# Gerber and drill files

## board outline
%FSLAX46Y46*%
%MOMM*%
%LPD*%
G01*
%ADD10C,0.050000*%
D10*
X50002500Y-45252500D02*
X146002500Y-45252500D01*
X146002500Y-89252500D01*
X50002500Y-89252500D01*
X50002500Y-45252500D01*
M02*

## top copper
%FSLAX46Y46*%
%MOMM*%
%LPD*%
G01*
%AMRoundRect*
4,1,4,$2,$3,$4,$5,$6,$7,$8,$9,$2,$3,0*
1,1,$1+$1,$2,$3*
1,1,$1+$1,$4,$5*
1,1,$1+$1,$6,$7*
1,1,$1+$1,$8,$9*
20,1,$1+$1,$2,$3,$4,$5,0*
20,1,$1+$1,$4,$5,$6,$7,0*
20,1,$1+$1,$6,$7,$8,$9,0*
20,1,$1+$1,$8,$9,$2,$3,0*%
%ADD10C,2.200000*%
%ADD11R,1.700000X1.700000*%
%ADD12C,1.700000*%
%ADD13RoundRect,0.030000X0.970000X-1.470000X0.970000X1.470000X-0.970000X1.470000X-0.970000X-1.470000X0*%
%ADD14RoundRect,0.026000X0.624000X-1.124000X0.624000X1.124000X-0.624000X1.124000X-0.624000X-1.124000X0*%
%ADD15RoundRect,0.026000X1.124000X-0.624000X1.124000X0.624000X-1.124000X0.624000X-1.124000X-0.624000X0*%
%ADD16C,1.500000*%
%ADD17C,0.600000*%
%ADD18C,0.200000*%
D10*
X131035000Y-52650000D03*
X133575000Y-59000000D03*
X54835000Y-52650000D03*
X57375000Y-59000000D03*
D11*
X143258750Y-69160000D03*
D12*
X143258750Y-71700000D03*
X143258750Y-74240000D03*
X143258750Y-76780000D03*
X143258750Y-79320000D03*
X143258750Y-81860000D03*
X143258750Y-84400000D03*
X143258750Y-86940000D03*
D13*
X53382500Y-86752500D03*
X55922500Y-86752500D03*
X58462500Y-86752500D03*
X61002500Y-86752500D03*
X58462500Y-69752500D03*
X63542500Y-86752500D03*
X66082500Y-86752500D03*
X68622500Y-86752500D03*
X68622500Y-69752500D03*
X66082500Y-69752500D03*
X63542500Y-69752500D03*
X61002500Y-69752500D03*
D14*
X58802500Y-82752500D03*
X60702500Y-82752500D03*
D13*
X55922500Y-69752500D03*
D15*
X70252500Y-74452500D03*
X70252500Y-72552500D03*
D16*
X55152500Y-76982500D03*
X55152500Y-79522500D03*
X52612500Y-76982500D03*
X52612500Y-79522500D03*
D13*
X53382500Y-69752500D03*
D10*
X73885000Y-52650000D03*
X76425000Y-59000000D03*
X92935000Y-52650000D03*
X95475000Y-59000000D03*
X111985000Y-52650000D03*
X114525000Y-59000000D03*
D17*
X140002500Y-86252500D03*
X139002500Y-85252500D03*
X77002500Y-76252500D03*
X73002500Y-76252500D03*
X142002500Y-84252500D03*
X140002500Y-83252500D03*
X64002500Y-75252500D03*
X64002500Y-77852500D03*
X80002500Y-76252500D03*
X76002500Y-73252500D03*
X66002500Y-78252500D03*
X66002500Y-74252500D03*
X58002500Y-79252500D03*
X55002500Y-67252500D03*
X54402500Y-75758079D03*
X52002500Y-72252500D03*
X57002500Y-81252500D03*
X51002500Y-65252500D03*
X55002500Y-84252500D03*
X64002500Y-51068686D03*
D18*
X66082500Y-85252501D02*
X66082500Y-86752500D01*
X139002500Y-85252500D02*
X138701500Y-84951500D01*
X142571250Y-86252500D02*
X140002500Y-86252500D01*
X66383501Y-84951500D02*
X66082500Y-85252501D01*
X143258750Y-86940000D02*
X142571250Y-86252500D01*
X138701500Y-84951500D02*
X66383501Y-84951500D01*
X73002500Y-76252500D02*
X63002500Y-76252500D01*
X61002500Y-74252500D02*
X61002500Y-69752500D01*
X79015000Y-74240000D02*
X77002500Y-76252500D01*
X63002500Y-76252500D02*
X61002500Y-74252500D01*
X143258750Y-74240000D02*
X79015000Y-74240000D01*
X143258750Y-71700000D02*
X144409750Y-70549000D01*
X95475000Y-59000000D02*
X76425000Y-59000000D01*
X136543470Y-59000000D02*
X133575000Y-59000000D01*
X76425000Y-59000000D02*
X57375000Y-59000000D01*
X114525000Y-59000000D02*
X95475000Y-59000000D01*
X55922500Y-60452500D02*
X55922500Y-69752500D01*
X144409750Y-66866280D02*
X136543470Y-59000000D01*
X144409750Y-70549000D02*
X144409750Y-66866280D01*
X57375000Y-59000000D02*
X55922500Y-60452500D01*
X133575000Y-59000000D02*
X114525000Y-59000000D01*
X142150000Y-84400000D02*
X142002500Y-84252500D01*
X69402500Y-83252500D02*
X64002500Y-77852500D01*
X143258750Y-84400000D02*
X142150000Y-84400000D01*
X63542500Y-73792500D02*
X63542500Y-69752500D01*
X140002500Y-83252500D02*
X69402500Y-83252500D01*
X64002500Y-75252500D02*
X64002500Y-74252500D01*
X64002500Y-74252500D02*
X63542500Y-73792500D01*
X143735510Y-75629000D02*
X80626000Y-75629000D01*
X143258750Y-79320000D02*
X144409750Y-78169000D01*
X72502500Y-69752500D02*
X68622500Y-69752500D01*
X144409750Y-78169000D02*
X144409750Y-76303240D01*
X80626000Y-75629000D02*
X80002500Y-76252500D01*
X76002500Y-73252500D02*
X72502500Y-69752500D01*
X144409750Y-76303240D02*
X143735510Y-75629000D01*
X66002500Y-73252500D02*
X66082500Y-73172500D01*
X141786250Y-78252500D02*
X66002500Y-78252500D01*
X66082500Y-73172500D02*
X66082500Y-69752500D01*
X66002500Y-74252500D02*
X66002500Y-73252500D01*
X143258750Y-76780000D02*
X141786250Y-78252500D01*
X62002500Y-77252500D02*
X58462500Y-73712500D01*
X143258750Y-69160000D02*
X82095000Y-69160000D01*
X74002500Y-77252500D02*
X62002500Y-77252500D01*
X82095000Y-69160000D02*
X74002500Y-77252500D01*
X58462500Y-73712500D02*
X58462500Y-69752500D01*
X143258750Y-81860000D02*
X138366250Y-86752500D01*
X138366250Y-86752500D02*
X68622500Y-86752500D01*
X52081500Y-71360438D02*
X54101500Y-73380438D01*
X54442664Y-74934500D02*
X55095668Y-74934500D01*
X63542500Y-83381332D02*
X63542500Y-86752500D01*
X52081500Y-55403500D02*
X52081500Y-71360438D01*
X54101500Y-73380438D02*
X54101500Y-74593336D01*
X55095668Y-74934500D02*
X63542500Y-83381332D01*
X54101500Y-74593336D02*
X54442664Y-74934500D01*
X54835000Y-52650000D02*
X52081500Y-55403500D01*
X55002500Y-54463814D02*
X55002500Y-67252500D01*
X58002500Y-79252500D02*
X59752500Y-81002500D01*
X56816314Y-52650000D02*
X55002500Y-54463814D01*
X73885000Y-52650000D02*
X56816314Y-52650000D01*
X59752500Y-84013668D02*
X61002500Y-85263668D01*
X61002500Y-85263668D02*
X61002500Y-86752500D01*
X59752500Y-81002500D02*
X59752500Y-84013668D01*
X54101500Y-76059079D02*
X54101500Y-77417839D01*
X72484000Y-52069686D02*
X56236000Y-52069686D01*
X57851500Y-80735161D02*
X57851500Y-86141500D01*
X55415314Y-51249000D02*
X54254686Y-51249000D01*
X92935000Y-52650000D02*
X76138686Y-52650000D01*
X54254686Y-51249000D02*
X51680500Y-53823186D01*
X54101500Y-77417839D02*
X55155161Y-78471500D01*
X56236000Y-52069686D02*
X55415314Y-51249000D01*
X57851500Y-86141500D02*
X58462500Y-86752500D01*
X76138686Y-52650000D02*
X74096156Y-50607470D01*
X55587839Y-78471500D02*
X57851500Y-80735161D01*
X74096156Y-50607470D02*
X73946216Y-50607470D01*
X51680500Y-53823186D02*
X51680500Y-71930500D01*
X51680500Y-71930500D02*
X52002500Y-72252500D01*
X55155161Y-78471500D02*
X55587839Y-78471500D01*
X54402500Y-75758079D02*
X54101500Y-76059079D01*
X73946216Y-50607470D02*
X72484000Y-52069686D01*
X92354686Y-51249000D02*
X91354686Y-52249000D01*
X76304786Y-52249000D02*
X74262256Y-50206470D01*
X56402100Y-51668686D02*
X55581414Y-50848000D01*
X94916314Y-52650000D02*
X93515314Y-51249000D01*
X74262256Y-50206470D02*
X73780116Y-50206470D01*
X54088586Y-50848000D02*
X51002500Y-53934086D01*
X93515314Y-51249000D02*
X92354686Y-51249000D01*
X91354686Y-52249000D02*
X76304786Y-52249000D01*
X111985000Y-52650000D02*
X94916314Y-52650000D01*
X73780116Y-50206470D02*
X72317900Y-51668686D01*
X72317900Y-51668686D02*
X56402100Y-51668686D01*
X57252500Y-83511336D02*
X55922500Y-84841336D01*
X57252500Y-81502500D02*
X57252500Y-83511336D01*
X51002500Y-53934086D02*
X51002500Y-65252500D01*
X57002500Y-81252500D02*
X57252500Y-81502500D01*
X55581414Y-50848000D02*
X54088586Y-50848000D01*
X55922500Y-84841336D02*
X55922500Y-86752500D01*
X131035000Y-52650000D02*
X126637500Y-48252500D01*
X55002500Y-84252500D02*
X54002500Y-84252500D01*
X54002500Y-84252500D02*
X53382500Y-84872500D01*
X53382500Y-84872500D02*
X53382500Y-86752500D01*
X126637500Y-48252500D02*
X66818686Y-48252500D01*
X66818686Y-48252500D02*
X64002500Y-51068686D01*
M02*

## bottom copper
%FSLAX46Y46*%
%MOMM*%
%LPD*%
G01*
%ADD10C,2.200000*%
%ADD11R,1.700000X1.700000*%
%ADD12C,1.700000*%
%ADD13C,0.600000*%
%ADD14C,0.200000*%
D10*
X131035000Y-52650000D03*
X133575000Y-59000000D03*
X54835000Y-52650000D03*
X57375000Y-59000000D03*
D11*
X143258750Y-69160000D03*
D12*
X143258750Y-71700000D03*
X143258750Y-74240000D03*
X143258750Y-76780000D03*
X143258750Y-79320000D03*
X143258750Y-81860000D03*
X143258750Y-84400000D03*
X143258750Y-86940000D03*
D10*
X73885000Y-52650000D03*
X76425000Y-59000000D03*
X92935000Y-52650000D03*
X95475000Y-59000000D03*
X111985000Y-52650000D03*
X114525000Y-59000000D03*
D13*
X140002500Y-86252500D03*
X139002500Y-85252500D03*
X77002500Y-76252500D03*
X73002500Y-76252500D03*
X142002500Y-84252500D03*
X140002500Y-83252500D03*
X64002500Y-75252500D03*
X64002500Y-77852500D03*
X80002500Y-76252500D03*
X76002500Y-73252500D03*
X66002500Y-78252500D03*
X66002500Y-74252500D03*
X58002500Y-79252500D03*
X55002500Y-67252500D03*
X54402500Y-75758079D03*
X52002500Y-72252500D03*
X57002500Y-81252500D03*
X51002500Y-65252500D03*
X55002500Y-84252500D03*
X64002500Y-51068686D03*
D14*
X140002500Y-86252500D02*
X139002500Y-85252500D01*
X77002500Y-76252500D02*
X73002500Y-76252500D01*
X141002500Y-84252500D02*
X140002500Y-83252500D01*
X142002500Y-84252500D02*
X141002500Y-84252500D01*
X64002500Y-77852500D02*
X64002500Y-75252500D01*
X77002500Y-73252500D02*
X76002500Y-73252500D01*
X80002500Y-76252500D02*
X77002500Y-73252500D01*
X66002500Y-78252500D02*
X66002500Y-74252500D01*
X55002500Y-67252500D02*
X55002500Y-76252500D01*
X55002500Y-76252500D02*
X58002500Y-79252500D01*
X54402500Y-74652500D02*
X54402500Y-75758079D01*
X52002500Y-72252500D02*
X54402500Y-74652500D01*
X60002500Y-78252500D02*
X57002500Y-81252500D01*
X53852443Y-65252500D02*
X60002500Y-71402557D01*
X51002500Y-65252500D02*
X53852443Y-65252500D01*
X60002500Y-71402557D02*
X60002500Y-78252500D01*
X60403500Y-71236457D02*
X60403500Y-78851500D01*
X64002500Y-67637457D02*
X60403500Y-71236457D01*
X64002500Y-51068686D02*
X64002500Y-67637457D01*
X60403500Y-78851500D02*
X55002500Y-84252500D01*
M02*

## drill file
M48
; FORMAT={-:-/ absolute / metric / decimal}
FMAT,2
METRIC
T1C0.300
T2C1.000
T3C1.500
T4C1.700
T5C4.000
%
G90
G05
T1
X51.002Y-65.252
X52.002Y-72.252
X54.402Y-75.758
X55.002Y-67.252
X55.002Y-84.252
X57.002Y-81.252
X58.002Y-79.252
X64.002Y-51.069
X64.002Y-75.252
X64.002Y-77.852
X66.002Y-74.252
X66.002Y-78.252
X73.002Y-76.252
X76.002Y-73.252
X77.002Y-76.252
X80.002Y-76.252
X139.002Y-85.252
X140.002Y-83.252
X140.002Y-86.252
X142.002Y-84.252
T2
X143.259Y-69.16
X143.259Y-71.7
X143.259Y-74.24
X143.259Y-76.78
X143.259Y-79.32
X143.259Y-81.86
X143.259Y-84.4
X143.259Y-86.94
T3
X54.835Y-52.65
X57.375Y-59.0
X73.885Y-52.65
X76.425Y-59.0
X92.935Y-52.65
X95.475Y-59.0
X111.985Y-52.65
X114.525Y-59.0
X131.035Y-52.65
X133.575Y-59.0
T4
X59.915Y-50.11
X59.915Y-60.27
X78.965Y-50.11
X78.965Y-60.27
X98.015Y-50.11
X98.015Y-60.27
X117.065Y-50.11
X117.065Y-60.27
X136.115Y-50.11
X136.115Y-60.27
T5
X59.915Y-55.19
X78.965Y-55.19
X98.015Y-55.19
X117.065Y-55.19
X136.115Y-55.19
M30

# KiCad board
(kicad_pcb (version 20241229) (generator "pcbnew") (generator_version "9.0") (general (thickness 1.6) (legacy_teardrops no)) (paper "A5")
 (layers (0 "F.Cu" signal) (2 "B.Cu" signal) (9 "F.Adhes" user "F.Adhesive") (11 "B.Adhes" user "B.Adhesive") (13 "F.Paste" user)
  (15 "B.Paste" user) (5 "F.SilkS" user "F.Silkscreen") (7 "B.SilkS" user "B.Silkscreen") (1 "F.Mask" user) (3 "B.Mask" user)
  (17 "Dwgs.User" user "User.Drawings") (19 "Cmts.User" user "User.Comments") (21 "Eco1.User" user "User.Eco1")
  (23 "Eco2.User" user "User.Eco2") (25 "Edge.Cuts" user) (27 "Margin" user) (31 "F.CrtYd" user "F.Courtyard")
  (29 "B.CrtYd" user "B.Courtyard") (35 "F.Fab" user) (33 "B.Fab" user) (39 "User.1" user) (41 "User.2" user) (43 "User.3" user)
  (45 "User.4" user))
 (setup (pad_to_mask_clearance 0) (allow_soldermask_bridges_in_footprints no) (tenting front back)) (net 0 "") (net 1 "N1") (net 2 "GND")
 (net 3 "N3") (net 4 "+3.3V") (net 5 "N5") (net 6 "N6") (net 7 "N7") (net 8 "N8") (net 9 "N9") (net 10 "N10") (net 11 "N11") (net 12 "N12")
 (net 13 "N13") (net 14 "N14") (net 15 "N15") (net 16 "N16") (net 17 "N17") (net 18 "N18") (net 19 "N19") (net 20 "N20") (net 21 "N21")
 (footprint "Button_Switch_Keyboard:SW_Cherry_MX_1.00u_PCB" (layer "F.Cu") (at 131.035 52.65 90)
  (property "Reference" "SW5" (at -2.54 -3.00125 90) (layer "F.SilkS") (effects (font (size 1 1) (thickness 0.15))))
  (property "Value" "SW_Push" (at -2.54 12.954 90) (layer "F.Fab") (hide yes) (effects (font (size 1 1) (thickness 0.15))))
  (pad "" np_thru_hole circle (at -7.62 5.08 90) (size 1.7 1.7) (drill 1.7) (layers "*.Cu" "*.Mask"))
  (pad "" np_thru_hole circle (at -2.54 5.08 90) (size 4 4) (drill 4) (layers "*.Cu" "*.Mask"))
  (pad "" np_thru_hole circle (at 2.54 5.08 90) (size 1.7 1.7) (drill 1.7) (layers "*.Cu" "*.Mask"))
  (pad "1" thru_hole circle (at 0 0 90) (size 2.2 2.2) (drill 1.5) (layers "*.Cu" "*.Mask") (remove_unused_layers no) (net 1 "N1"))
  (pad "2" thru_hole circle (at -6.35 2.54 90) (size 2.2 2.2) (drill 1.5) (layers "*.Cu" "*.Mask") (remove_unused_layers no) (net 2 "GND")))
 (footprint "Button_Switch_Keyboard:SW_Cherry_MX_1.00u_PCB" (layer "F.Cu") (at 54.835 52.65 90)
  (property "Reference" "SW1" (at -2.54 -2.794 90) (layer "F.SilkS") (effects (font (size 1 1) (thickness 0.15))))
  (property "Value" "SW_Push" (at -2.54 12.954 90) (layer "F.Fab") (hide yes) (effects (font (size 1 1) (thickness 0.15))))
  (pad "" np_thru_hole circle (at -7.62 5.08 90) (size 1.7 1.7) (drill 1.7) (layers "*.Cu" "*.Mask"))
  (pad "" np_thru_hole circle (at -2.54 5.08 90) (size 4 4) (drill 4) (layers "*.Cu" "*.Mask"))
  (pad "" np_thru_hole circle (at 2.54 5.08 90) (size 1.7 1.7) (drill 1.7) (layers "*.Cu" "*.Mask"))
  (pad "1" thru_hole circle (at 0 0 90) (size 2.2 2.2) (drill 1.5) (layers "*.Cu" "*.Mask") (remove_unused_layers no) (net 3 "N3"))
  (pad "2" thru_hole circle (at -6.35 2.54 90) (size 2.2 2.2) (drill 1.5) (layers "*.Cu" "*.Mask") (remove_unused_layers no) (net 2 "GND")))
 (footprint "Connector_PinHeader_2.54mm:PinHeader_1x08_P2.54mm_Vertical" (layer "F.Cu") (at 143.25875 69.16)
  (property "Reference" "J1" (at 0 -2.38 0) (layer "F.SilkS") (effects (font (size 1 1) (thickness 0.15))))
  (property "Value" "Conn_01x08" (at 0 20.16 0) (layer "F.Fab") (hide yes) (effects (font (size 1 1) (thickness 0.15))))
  (pad "1" thru_hole rect (at 0 0) (size 1.7 1.7) (drill 1) (layers "*.Cu" "*.Mask") (remove_unused_layers no) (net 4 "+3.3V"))
  (pad "2" thru_hole circle (at 0 2.54) (size 1.7 1.7) (drill 1) (layers "*.Cu" "*.Mask") (remove_unused_layers no) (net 2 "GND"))
  (pad "3" thru_hole circle (at 0 5.08) (size 1.7 1.7) (drill 1) (layers "*.Cu" "*.Mask") (remove_unused_layers no) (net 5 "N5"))
  (pad "4" thru_hole circle (at 0 7.62) (size 1.7 1.7) (drill 1) (layers "*.Cu" "*.Mask") (remove_unused_layers no) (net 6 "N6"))
  (pad "5" thru_hole circle (at 0 10.16) (size 1.7 1.7) (drill 1) (layers "*.Cu" "*.Mask") (remove_unused_layers no) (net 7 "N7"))
  (pad "6" thru_hole circle (at 0 12.7) (size 1.7 1.7) (drill 1) (layers "*.Cu" "*.Mask") (remove_unused_layers no) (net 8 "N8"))
  (pad "7" thru_hole circle (at 0 15.24) (size 1.7 1.7) (drill 1) (layers "*.Cu" "*.Mask") (remove_unused_layers no) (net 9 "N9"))
  (pad "8" thru_hole circle (at 0 17.78) (size 1.7 1.7) (drill 1) (layers "*.Cu" "*.Mask") (remove_unused_layers no) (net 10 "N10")))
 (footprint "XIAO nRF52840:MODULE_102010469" (layer "F.Cu") (at 61.0025 78.2525 90)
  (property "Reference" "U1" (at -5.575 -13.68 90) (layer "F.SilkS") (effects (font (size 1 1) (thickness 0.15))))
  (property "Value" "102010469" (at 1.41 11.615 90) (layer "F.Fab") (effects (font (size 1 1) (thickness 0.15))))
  (pad "0" smd roundrect (at -8.5 -7.62 90) (size 3 2) (layers "F.Cu" "F.Mask" "F.Paste") (roundrect_rratio 0.015) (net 1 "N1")
   (solder_mask_margin 0.102))
  (pad "1" smd roundrect (at -8.5 -5.08 90) (size 3 2) (layers "F.Cu" "F.Mask" "F.Paste") (roundrect_rratio 0.015) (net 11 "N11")
   (solder_mask_margin 0.102))
  (pad "2" smd roundrect (at -8.5 -2.54 90) (size 3 2) (layers "F.Cu" "F.Mask" "F.Paste") (roundrect_rratio 0.015) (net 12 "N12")
   (solder_mask_margin 0.102))
  (pad "3" smd roundrect (at -8.5 0 90) (size 3 2) (layers "F.Cu" "F.Mask" "F.Paste") (roundrect_rratio 0.015) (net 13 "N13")
   (solder_mask_margin 0.102))
  (pad "3V3" smd roundrect (at 8.5 -2.54 90) (size 3 2) (layers "F.Cu" "F.Mask" "F.Paste") (roundrect_rratio 0.015) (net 4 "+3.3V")
   (solder_mask_margin 0.102))
  (pad "4" smd roundrect (at -8.5 2.54 90) (size 3 2) (layers "F.Cu" "F.Mask" "F.Paste") (roundrect_rratio 0.015) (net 3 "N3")
   (solder_mask_margin 0.102))
  (pad "5" smd roundrect (at -8.5 5.08 90) (size 3 2) (layers "F.Cu" "F.Mask" "F.Paste") (roundrect_rratio 0.015) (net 10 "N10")
   (solder_mask_margin 0.102))
  (pad "6" smd roundrect (at -8.5 7.62 90) (size 3 2) (layers "F.Cu" "F.Mask" "F.Paste") (roundrect_rratio 0.015) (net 8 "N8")
   (solder_mask_margin 0.102))
  (pad "7" smd roundrect (at 8.5 7.62 90) (size 3 2) (layers "F.Cu" "F.Mask" "F.Paste") (roundrect_rratio 0.015) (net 7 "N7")
   (solder_mask_margin 0.102))
  (pad "8" smd roundrect (at 8.5 5.08 90) (size 3 2) (layers "F.Cu" "F.Mask" "F.Paste") (roundrect_rratio 0.015) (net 6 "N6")
   (solder_mask_margin 0.102))
  (pad "9" smd roundrect (at 8.5 2.54 90) (size 3 2) (layers "F.Cu" "F.Mask" "F.Paste") (roundrect_rratio 0.015) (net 9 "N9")
   (solder_mask_margin 0.102))
  (pad "10" smd roundrect (at 8.5 0 90) (size 3 2) (layers "F.Cu" "F.Mask" "F.Paste") (roundrect_rratio 0.015) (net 5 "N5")
   (solder_mask_margin 0.102))
  (pad "BAT_N" smd roundrect (at -4.5 -2.2 90) (size 2.3 1.3) (layers "F.Cu" "F.Mask" "F.Paste") (roundrect_rratio 0.02) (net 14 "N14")
   (solder_mask_margin 0.102))
  (pad "BAT_P" smd roundrect (at -4.5 -0.3 90) (size 2.3 1.3) (layers "F.Cu" "F.Mask" "F.Paste") (roundrect_rratio 0.02) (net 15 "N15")
   (solder_mask_margin 0.102))
  (pad "GND" smd roundrect (at 8.5 -5.08 90) (size 3 2) (layers "F.Cu" "F.Mask" "F.Paste") (roundrect_rratio 0.015) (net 2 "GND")
   (solder_mask_margin 0.102))
  (pad "NFC1" smd roundrect (at 3.8 9.25 90) (size 1.3 2.3) (layers "F.Cu" "F.Mask" "F.Paste") (roundrect_rratio 0.02) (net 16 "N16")
   (solder_mask_margin 0.102))
  (pad "NFC2" smd roundrect (at 5.7 9.25 90) (size 1.3 2.3) (layers "F.Cu" "F.Mask" "F.Paste") (roundrect_rratio 0.02) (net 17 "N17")
   (solder_mask_margin 0.102))
  (pad "TP1" smd circle (at 1.27 -5.85 90) (size 1.5 1.5) (layers "F.Cu" "F.Mask" "F.Paste") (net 2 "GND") (solder_mask_margin 0.102))
  (pad "TP2" smd circle (at -1.27 -5.85 90) (size 1.5 1.5) (layers "F.Cu" "F.Mask" "F.Paste") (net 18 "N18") (solder_mask_margin 0.102))
  (pad "TP3" smd circle (at 1.27 -8.39 90) (size 1.5 1.5) (layers "F.Cu" "F.Mask" "F.Paste") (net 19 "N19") (solder_mask_margin 0.102))
  (pad "TP5" smd circle (at -1.27 -8.39 90) (size 1.5 1.5) (layers "F.Cu" "F.Mask" "F.Paste") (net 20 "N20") (solder_mask_margin 0.102))
  (pad "VUSB" smd roundrect (at 8.5 -7.62 90) (size 3 2) (layers "F.Cu" "F.Mask" "F.Paste") (roundrect_rratio 0.015) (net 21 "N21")
   (solder_mask_margin 0.102))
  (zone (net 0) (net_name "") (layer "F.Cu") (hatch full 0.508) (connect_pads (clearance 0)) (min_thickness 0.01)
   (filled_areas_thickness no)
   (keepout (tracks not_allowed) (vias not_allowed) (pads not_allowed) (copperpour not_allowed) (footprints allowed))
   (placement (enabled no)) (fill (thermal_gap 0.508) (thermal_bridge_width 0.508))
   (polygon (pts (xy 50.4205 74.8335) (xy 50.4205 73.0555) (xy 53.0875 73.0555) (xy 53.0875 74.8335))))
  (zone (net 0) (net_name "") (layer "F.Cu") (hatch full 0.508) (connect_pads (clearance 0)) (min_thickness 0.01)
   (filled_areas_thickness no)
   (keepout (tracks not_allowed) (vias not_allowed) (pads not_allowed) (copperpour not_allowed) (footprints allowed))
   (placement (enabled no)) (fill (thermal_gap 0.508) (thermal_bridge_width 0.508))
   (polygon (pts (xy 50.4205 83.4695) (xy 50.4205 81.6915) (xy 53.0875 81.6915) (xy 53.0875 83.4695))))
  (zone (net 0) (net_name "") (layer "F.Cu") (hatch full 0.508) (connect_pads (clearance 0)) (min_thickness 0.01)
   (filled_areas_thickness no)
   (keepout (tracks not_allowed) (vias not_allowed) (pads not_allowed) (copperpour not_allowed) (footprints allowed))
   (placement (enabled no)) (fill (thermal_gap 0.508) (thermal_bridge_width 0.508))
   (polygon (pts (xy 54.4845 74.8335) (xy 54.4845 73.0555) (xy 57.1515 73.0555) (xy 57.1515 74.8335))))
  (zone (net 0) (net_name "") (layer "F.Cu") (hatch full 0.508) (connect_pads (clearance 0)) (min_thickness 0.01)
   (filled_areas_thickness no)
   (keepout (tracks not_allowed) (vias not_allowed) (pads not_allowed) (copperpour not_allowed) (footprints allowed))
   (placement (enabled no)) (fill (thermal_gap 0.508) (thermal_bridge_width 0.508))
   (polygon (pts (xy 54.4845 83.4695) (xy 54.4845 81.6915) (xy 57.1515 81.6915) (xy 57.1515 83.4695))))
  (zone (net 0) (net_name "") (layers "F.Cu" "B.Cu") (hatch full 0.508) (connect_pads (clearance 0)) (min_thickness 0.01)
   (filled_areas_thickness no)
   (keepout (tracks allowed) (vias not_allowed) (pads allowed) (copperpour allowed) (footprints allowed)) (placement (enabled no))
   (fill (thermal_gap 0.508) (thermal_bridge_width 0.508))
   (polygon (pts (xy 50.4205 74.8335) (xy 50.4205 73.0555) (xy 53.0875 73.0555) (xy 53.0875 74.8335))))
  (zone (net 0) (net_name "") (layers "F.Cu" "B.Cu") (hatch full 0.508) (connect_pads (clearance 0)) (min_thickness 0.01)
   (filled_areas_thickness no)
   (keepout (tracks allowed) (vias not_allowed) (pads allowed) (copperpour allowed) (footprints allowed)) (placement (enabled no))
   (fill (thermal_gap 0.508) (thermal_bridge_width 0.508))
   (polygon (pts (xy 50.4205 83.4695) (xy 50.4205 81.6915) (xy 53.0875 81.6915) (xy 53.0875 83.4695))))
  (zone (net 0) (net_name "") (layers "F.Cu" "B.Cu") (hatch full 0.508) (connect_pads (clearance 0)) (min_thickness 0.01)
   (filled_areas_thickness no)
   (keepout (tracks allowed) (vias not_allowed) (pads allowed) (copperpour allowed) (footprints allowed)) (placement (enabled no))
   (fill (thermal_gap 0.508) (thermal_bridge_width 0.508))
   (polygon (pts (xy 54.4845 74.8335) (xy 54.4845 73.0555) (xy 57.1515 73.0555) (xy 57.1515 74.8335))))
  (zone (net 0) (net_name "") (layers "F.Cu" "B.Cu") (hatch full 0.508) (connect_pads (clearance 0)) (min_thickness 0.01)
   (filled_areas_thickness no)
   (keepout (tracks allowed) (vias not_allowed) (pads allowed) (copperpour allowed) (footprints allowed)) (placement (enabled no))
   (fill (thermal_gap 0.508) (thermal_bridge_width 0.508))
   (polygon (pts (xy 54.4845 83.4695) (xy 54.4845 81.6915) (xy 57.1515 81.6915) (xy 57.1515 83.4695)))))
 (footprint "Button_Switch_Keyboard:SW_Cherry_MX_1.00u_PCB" (layer "F.Cu") (at 73.885 52.65 90)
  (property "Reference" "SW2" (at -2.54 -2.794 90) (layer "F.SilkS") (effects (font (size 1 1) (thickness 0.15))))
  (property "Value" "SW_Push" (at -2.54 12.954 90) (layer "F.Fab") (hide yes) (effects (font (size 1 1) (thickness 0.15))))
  (pad "" np_thru_hole circle (at -7.62 5.08 90) (size 1.7 1.7) (drill 1.7) (layers "*.Cu" "*.Mask"))
  (pad "" np_thru_hole circle (at -2.54 5.08 90) (size 4 4) (drill 4) (layers "*.Cu" "*.Mask"))
  (pad "" np_thru_hole circle (at 2.54 5.08 90) (size 1.7 1.7) (drill 1.7) (layers "*.Cu" "*.Mask"))
  (pad "1" thru_hole circle (at 0 0 90) (size 2.2 2.2) (drill 1.5) (layers "*.Cu" "*.Mask") (remove_unused_layers no) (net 13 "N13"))
  (pad "2" thru_hole circle (at -6.35 2.54 90) (size 2.2 2.2) (drill 1.5) (layers "*.Cu" "*.Mask") (remove_unused_layers no) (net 2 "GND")))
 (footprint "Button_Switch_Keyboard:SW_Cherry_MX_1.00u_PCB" (layer "F.Cu") (at 92.935 52.65 90)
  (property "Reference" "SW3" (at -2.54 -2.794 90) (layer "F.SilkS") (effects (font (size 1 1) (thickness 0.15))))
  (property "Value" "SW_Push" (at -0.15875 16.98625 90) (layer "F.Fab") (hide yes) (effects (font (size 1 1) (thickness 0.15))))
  (pad "" np_thru_hole circle (at -7.62 5.08 90) (size 1.7 1.7) (drill 1.7) (layers "*.Cu" "*.Mask"))
  (pad "" np_thru_hole circle (at -2.54 5.08 90) (size 4 4) (drill 4) (layers "*.Cu" "*.Mask"))
  (pad "" np_thru_hole circle (at 2.54 5.08 90) (size 1.7 1.7) (drill 1.7) (layers "*.Cu" "*.Mask"))
  (pad "1" thru_hole circle (at 0 0 90) (size 2.2 2.2) (drill 1.5) (layers "*.Cu" "*.Mask") (remove_unused_layers no) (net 12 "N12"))
  (pad "2" thru_hole circle (at -6.35 2.54 90) (size 2.2 2.2) (drill 1.5) (layers "*.Cu" "*.Mask") (remove_unused_layers no) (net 2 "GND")))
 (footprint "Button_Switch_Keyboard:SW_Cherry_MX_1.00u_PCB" (layer "F.Cu") (at 111.985 52.65 90)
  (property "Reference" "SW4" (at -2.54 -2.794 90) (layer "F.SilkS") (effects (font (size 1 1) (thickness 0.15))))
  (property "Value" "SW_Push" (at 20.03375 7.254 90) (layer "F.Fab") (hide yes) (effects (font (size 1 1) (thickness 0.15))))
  (pad "" np_thru_hole circle (at -7.62 5.08 90) (size 1.7 1.7) (drill 1.7) (layers "*.Cu" "*.Mask"))
  (pad "" np_thru_hole circle (at -2.54 5.08 90) (size 4 4) (drill 4) (layers "*.Cu" "*.Mask"))
  (pad "" np_thru_hole circle (at 2.54 5.08 90) (size 1.7 1.7) (drill 1.7) (layers "*.Cu" "*.Mask"))
  (pad "1" thru_hole circle (at 0 0 90) (size 2.2 2.2) (drill 1.5) (layers "*.Cu" "*.Mask") (remove_unused_layers no) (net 11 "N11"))
  (pad "2" thru_hole circle (at -6.35 2.54 90) (size 2.2 2.2) (drill 1.5) (layers "*.Cu" "*.Mask") (remove_unused_layers no) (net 2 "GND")))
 (gr_rect (start 50.0025 45.2525) (end 146.0025 89.2525) (stroke (width 0.05) (type default)) (fill no) (layer "Edge.Cuts"))
 (segment (start 66.0825 85.252501) (end 66.0825 86.7525) (width 0.2) (layer "F.Cu") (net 10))
 (segment (start 139.0025 85.2525) (end 138.7015 84.9515) (width 0.2) (layer "F.Cu") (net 10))
 (segment (start 142.57125 86.2525) (end 140.0025 86.2525) (width 0.2) (layer "F.Cu") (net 10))
 (segment (start 66.383501 84.9515) (end 66.0825 85.252501) (width 0.2) (layer "F.Cu") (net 10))
 (segment (start 143.25875 86.94) (end 142.57125 86.2525) (width 0.2) (layer "F.Cu") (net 10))
 (segment (start 138.7015 84.9515) (end 66.383501 84.9515) (width 0.2) (layer "F.Cu") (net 10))
 (via (at 140.0025 86.2525) (size 0.6) (drill 0.3) (layers "F.Cu" "B.Cu") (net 10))
 (via (at 139.0025 85.2525) (size 0.6) (drill 0.3) (layers "F.Cu" "B.Cu") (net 10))
 (segment (start 140.0025 86.2525) (end 139.0025 85.2525) (width 0.2) (layer "B.Cu") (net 10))
 (segment (start 73.0025 76.2525) (end 63.0025 76.2525) (width 0.2) (layer "F.Cu") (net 5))
 (segment (start 61.0025 74.2525) (end 61.0025 69.7525) (width 0.2) (layer "F.Cu") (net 5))
 (segment (start 79.015 74.24) (end 77.0025 76.2525) (width 0.2) (layer "F.Cu") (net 5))
 (segment (start 63.0025 76.2525) (end 61.0025 74.2525) (width 0.2) (layer "F.Cu") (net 5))
 (segment (start 143.25875 74.24) (end 79.015 74.24) (width 0.2) (layer "F.Cu") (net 5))
 (via (at 77.0025 76.2525) (size 0.6) (drill 0.3) (layers "F.Cu" "B.Cu") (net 5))
 (via (at 73.0025 76.2525) (size 0.6) (drill 0.3) (layers "F.Cu" "B.Cu") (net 5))
 (segment (start 77.0025 76.2525) (end 73.0025 76.2525) (width 0.2) (layer "B.Cu") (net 5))
 (segment (start 143.25875 71.7) (end 144.40975 70.549) (width 0.2) (layer "F.Cu") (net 2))
 (segment (start 95.475 59) (end 76.425 59) (width 0.2) (layer "F.Cu") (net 2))
 (segment (start 136.54347 59) (end 133.575 59) (width 0.2) (layer "F.Cu") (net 2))
 (segment (start 76.425 59) (end 57.375 59) (width 0.2) (layer "F.Cu") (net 2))
 (segment (start 114.525 59) (end 95.475 59) (width 0.2) (layer "F.Cu") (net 2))
 (segment (start 55.9225 60.4525) (end 55.9225 69.7525) (width 0.2) (layer "F.Cu") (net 2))
 (segment (start 144.40975 66.86628) (end 136.54347 59) (width 0.2) (layer "F.Cu") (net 2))
 (segment (start 144.40975 70.549) (end 144.40975 66.86628) (width 0.2) (layer "F.Cu") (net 2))
 (segment (start 57.375 59) (end 55.9225 60.4525) (width 0.2) (layer "F.Cu") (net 2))
 (segment (start 133.575 59) (end 114.525 59) (width 0.2) (layer "F.Cu") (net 2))
 (segment (start 142.15 84.4) (end 142.0025 84.2525) (width 0.2) (layer "F.Cu") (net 9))
 (segment (start 69.4025 83.2525) (end 64.0025 77.8525) (width 0.2) (layer "F.Cu") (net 9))
 (segment (start 143.25875 84.4) (end 142.15 84.4) (width 0.2) (layer "F.Cu") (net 9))
 (segment (start 63.5425 73.7925) (end 63.5425 69.7525) (width 0.2) (layer "F.Cu") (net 9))
 (segment (start 140.0025 83.2525) (end 69.4025 83.2525) (width 0.2) (layer "F.Cu") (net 9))
 (segment (start 64.0025 75.2525) (end 64.0025 74.2525) (width 0.2) (layer "F.Cu") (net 9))
 (segment (start 64.0025 74.2525) (end 63.5425 73.7925) (width 0.2) (layer "F.Cu") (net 9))
 (via (at 142.0025 84.2525) (size 0.6) (drill 0.3) (layers "F.Cu" "B.Cu") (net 9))
 (via (at 140.0025 83.2525) (size 0.6) (drill 0.3) (layers "F.Cu" "B.Cu") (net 9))
 (via (at 64.0025 75.2525) (size 0.6) (drill 0.3) (layers "F.Cu" "B.Cu") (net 9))
 (via (at 64.0025 77.8525) (size 0.6) (drill 0.3) (layers "F.Cu" "B.Cu") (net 9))
 (segment (start 141.0025 84.2525) (end 140.0025 83.2525) (width 0.2) (layer "B.Cu") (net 9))
 (segment (start 142.0025 84.2525) (end 141.0025 84.2525) (width 0.2) (layer "B.Cu") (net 9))
 (segment (start 64.0025 77.8525) (end 64.0025 75.2525) (width 0.2) (layer "B.Cu") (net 9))
 (segment (start 143.73551 75.629) (end 80.626 75.629) (width 0.2) (layer "F.Cu") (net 7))
 (segment (start 143.25875 79.32) (end 144.40975 78.169) (width 0.2) (layer "F.Cu") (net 7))
 (segment (start 72.5025 69.7525) (end 68.6225 69.7525) (width 0.2) (layer "F.Cu") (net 7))
 (segment (start 144.40975 78.169) (end 144.40975 76.30324) (width 0.2) (layer "F.Cu") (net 7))
 (segment (start 80.626 75.629) (end 80.0025 76.2525) (width 0.2) (layer "F.Cu") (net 7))
 (segment (start 76.0025 73.2525) (end 72.5025 69.7525) (width 0.2) (layer "F.Cu") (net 7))
 (segment (start 144.40975 76.30324) (end 143.73551 75.629) (width 0.2) (layer "F.Cu") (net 7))
 (via (at 80.0025 76.2525) (size 0.6) (drill 0.3) (layers "F.Cu" "B.Cu") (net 7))
 (via (at 76.0025 73.2525) (size 0.6) (drill 0.3) (layers "F.Cu" "B.Cu") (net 7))
 (segment (start 77.0025 73.2525) (end 76.0025 73.2525) (width 0.2) (layer "B.Cu") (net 7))
 (segment (start 80.0025 76.2525) (end 77.0025 73.2525) (width 0.2) (layer "B.Cu") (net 7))
 (segment (start 66.0025 73.2525) (end 66.0825 73.1725) (width 0.2) (layer "F.Cu") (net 6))
 (segment (start 141.78625 78.2525) (end 66.0025 78.2525) (width 0.2) (layer "F.Cu") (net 6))
 (segment (start 66.0825 73.1725) (end 66.0825 69.7525) (width 0.2) (layer "F.Cu") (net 6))
 (segment (start 66.0025 74.2525) (end 66.0025 73.2525) (width 0.2) (layer "F.Cu") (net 6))
 (segment (start 143.25875 76.78) (end 141.78625 78.2525) (width 0.2) (layer "F.Cu") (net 6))
 (via (at 66.0025 78.2525) (size 0.6) (drill 0.3) (layers "F.Cu" "B.Cu") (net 6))
 (via (at 66.0025 74.2525) (size 0.6) (drill 0.3) (layers "F.Cu" "B.Cu") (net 6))
 (segment (start 66.0025 78.2525) (end 66.0025 74.2525) (width 0.2) (layer "B.Cu") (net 6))
 (segment (start 62.0025 77.2525) (end 58.4625 73.7125) (width 0.2) (layer "F.Cu") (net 4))
 (segment (start 143.25875 69.16) (end 82.095 69.16) (width 0.2) (layer "F.Cu") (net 4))
 (segment (start 74.0025 77.2525) (end 62.0025 77.2525) (width 0.2) (layer "F.Cu") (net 4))
 (segment (start 82.095 69.16) (end 74.0025 77.2525) (width 0.2) (layer "F.Cu") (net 4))
 (segment (start 58.4625 73.7125) (end 58.4625 69.7525) (width 0.2) (layer "F.Cu") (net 4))
 (segment (start 143.25875 81.86) (end 138.36625 86.7525) (width 0.2) (layer "F.Cu") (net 8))
 (segment (start 138.36625 86.7525) (end 68.6225 86.7525) (width 0.2) (layer "F.Cu") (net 8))
 (segment (start 52.0815 71.360438) (end 54.1015 73.380438) (width 0.2) (layer "F.Cu") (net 3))
 (segment (start 54.442664 74.9345) (end 55.095668 74.9345) (width 0.2) (layer "F.Cu") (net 3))
 (segment (start 63.5425 83.381332) (end 63.5425 86.7525) (width 0.2) (layer "F.Cu") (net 3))
 (segment (start 52.0815 55.4035) (end 52.0815 71.360438) (width 0.2) (layer "F.Cu") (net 3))
 (segment (start 54.1015 73.380438) (end 54.1015 74.593336) (width 0.2) (layer "F.Cu") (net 3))
 (segment (start 55.095668 74.9345) (end 63.5425 83.381332) (width 0.2) (layer "F.Cu") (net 3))
 (segment (start 54.1015 74.593336) (end 54.442664 74.9345) (width 0.2) (layer "F.Cu") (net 3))
 (segment (start 54.835 52.65) (end 52.0815 55.4035) (width 0.2) (layer "F.Cu") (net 3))
 (segment (start 55.0025 54.463814) (end 55.0025 67.2525) (width 0.2) (layer "F.Cu") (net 13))
 (segment (start 58.0025 79.2525) (end 59.7525 81.0025) (width 0.2) (layer "F.Cu") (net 13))
 (segment (start 56.816314 52.65) (end 55.0025 54.463814) (width 0.2) (layer "F.Cu") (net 13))
 (segment (start 73.885 52.65) (end 56.816314 52.65) (width 0.2) (layer "F.Cu") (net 13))
 (segment (start 59.7525 84.013668) (end 61.0025 85.263668) (width 0.2) (layer "F.Cu") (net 13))
 (segment (start 61.0025 85.263668) (end 61.0025 86.7525) (width 0.2) (layer "F.Cu") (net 13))
 (segment (start 59.7525 81.0025) (end 59.7525 84.013668) (width 0.2) (layer "F.Cu") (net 13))
 (via (at 58.0025 79.2525) (size 0.6) (drill 0.3) (layers "F.Cu" "B.Cu") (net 13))
 (via (at 55.0025 67.2525) (size 0.6) (drill 0.3) (layers "F.Cu" "B.Cu") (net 13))
 (segment (start 55.0025 67.2525) (end 55.0025 76.2525) (width 0.2) (layer "B.Cu") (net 13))
 (segment (start 55.0025 76.2525) (end 58.0025 79.2525) (width 0.2) (layer "B.Cu") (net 13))
 (segment (start 54.1015 76.059079) (end 54.1015 77.417839) (width 0.2) (layer "F.Cu") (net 12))
 (segment (start 72.484 52.069686) (end 56.236 52.069686) (width 0.2) (layer "F.Cu") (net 12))
 (segment (start 57.8515 80.735161) (end 57.8515 86.1415) (width 0.2) (layer "F.Cu") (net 12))
 (segment (start 55.415314 51.249) (end 54.254686 51.249) (width 0.2) (layer "F.Cu") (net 12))
 (segment (start 92.935 52.65) (end 76.138686 52.65) (width 0.2) (layer "F.Cu") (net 12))
 (segment (start 54.254686 51.249) (end 51.6805 53.823186) (width 0.2) (layer "F.Cu") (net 12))
 (segment (start 54.1015 77.417839) (end 55.155161 78.4715) (width 0.2) (layer "F.Cu") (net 12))
 (segment (start 56.236 52.069686) (end 55.415314 51.249) (width 0.2) (layer "F.Cu") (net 12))
 (segment (start 57.8515 86.1415) (end 58.4625 86.7525) (width 0.2) (layer "F.Cu") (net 12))
 (segment (start 76.138686 52.65) (end 74.096156 50.60747) (width 0.2) (layer "F.Cu") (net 12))
 (segment (start 55.587839 78.4715) (end 57.8515 80.735161) (width 0.2) (layer "F.Cu") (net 12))
 (segment (start 74.096156 50.60747) (end 73.946216 50.60747) (width 0.2) (layer "F.Cu") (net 12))
 (segment (start 51.6805 53.823186) (end 51.6805 71.9305) (width 0.2) (layer "F.Cu") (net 12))
 (segment (start 51.6805 71.9305) (end 52.0025 72.2525) (width 0.2) (layer "F.Cu") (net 12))
 (segment (start 55.155161 78.4715) (end 55.587839 78.4715) (width 0.2) (layer "F.Cu") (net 12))
 (segment (start 54.4025 75.758079) (end 54.1015 76.059079) (width 0.2) (layer "F.Cu") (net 12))
 (segment (start 73.946216 50.60747) (end 72.484 52.069686) (width 0.2) (layer "F.Cu") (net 12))
 (via (at 54.4025 75.758079) (size 0.6) (drill 0.3) (layers "F.Cu" "B.Cu") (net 12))
 (via (at 52.0025 72.2525) (size 0.6) (drill 0.3) (layers "F.Cu" "B.Cu") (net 12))
 (segment (start 54.4025 74.6525) (end 54.4025 75.758079) (width 0.2) (layer "B.Cu") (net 12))
 (segment (start 52.0025 72.2525) (end 54.4025 74.6525) (width 0.2) (layer "B.Cu") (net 12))
 (segment (start 92.354686 51.249) (end 91.354686 52.249) (width 0.2) (layer "F.Cu") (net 11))
 (segment (start 76.304786 52.249) (end 74.262256 50.20647) (width 0.2) (layer "F.Cu") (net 11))
 (segment (start 56.4021 51.668686) (end 55.581414 50.848) (width 0.2) (layer "F.Cu") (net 11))
 (segment (start 94.916314 52.65) (end 93.515314 51.249) (width 0.2) (layer "F.Cu") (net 11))
 (segment (start 74.262256 50.20647) (end 73.780116 50.20647) (width 0.2) (layer "F.Cu") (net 11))
 (segment (start 54.088586 50.848) (end 51.0025 53.934086) (width 0.2) (layer "F.Cu") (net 11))
 (segment (start 93.515314 51.249) (end 92.354686 51.249) (width 0.2) (layer "F.Cu") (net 11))
 (segment (start 91.354686 52.249) (end 76.304786 52.249) (width 0.2) (layer "F.Cu") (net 11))
 (segment (start 111.985 52.65) (end 94.916314 52.65) (width 0.2) (layer "F.Cu") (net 11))
 (segment (start 73.780116 50.20647) (end 72.3179 51.668686) (width 0.2) (layer "F.Cu") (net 11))
 (segment (start 72.3179 51.668686) (end 56.4021 51.668686) (width 0.2) (layer "F.Cu") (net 11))
 (segment (start 57.2525 83.511336) (end 55.9225 84.841336) (width 0.2) (layer "F.Cu") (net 11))
 (segment (start 57.2525 81.5025) (end 57.2525 83.511336) (width 0.2) (layer "F.Cu") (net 11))
 (segment (start 51.0025 53.934086) (end 51.0025 65.2525) (width 0.2) (layer "F.Cu") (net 11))
 (segment (start 57.0025 81.2525) (end 57.2525 81.5025) (width 0.2) (layer "F.Cu") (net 11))
 (segment (start 55.581414 50.848) (end 54.088586 50.848) (width 0.2) (layer "F.Cu") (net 11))
 (segment (start 55.9225 84.841336) (end 55.9225 86.7525) (width 0.2) (layer "F.Cu") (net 11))
 (via (at 57.0025 81.2525) (size 0.6) (drill 0.3) (layers "F.Cu" "B.Cu") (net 11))
 (via (at 51.0025 65.2525) (size 0.6) (drill 0.3) (layers "F.Cu" "B.Cu") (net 11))
 (segment (start 60.0025 78.2525) (end 57.0025 81.2525) (width 0.2) (layer "B.Cu") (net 11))
 (segment (start 53.852443 65.2525) (end 60.0025 71.402557) (width 0.2) (layer "B.Cu") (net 11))
 (segment (start 51.0025 65.2525) (end 53.852443 65.2525) (width 0.2) (layer "B.Cu") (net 11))
 (segment (start 60.0025 71.402557) (end 60.0025 78.2525) (width 0.2) (layer "B.Cu") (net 11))
 (segment (start 131.035 52.65) (end 126.6375 48.2525) (width 0.2) (layer "F.Cu") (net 1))
 (segment (start 55.0025 84.2525) (end 54.0025 84.2525) (width 0.2) (layer "F.Cu") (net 1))
 (segment (start 54.0025 84.2525) (end 53.3825 84.8725) (width 0.2) (layer "F.Cu") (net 1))
 (segment (start 53.3825 84.8725) (end 53.3825 86.7525) (width 0.2) (layer "F.Cu") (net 1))
 (segment (start 126.6375 48.2525) (end 66.818686 48.2525) (width 0.2) (layer "F.Cu") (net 1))
 (segment (start 66.818686 48.2525) (end 64.0025 51.068686) (width 0.2) (layer "F.Cu") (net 1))
 (via (at 55.0025 84.2525) (size 0.6) (drill 0.3) (layers "F.Cu" "B.Cu") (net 1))
 (via (at 64.0025 51.068686) (size 0.6) (drill 0.3) (layers "F.Cu" "B.Cu") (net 1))
 (segment (start 60.4035 71.236457) (end 60.4035 78.8515) (width 0.2) (layer "B.Cu") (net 1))
 (segment (start 64.0025 67.637457) (end 60.4035 71.236457) (width 0.2) (layer "B.Cu") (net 1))
 (segment (start 64.0025 51.068686) (end 64.0025 67.637457) (width 0.2) (layer "B.Cu") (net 1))
 (segment (start 60.4035 78.8515) (end 55.0025 84.2525) (width 0.2) (layer "B.Cu") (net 1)))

